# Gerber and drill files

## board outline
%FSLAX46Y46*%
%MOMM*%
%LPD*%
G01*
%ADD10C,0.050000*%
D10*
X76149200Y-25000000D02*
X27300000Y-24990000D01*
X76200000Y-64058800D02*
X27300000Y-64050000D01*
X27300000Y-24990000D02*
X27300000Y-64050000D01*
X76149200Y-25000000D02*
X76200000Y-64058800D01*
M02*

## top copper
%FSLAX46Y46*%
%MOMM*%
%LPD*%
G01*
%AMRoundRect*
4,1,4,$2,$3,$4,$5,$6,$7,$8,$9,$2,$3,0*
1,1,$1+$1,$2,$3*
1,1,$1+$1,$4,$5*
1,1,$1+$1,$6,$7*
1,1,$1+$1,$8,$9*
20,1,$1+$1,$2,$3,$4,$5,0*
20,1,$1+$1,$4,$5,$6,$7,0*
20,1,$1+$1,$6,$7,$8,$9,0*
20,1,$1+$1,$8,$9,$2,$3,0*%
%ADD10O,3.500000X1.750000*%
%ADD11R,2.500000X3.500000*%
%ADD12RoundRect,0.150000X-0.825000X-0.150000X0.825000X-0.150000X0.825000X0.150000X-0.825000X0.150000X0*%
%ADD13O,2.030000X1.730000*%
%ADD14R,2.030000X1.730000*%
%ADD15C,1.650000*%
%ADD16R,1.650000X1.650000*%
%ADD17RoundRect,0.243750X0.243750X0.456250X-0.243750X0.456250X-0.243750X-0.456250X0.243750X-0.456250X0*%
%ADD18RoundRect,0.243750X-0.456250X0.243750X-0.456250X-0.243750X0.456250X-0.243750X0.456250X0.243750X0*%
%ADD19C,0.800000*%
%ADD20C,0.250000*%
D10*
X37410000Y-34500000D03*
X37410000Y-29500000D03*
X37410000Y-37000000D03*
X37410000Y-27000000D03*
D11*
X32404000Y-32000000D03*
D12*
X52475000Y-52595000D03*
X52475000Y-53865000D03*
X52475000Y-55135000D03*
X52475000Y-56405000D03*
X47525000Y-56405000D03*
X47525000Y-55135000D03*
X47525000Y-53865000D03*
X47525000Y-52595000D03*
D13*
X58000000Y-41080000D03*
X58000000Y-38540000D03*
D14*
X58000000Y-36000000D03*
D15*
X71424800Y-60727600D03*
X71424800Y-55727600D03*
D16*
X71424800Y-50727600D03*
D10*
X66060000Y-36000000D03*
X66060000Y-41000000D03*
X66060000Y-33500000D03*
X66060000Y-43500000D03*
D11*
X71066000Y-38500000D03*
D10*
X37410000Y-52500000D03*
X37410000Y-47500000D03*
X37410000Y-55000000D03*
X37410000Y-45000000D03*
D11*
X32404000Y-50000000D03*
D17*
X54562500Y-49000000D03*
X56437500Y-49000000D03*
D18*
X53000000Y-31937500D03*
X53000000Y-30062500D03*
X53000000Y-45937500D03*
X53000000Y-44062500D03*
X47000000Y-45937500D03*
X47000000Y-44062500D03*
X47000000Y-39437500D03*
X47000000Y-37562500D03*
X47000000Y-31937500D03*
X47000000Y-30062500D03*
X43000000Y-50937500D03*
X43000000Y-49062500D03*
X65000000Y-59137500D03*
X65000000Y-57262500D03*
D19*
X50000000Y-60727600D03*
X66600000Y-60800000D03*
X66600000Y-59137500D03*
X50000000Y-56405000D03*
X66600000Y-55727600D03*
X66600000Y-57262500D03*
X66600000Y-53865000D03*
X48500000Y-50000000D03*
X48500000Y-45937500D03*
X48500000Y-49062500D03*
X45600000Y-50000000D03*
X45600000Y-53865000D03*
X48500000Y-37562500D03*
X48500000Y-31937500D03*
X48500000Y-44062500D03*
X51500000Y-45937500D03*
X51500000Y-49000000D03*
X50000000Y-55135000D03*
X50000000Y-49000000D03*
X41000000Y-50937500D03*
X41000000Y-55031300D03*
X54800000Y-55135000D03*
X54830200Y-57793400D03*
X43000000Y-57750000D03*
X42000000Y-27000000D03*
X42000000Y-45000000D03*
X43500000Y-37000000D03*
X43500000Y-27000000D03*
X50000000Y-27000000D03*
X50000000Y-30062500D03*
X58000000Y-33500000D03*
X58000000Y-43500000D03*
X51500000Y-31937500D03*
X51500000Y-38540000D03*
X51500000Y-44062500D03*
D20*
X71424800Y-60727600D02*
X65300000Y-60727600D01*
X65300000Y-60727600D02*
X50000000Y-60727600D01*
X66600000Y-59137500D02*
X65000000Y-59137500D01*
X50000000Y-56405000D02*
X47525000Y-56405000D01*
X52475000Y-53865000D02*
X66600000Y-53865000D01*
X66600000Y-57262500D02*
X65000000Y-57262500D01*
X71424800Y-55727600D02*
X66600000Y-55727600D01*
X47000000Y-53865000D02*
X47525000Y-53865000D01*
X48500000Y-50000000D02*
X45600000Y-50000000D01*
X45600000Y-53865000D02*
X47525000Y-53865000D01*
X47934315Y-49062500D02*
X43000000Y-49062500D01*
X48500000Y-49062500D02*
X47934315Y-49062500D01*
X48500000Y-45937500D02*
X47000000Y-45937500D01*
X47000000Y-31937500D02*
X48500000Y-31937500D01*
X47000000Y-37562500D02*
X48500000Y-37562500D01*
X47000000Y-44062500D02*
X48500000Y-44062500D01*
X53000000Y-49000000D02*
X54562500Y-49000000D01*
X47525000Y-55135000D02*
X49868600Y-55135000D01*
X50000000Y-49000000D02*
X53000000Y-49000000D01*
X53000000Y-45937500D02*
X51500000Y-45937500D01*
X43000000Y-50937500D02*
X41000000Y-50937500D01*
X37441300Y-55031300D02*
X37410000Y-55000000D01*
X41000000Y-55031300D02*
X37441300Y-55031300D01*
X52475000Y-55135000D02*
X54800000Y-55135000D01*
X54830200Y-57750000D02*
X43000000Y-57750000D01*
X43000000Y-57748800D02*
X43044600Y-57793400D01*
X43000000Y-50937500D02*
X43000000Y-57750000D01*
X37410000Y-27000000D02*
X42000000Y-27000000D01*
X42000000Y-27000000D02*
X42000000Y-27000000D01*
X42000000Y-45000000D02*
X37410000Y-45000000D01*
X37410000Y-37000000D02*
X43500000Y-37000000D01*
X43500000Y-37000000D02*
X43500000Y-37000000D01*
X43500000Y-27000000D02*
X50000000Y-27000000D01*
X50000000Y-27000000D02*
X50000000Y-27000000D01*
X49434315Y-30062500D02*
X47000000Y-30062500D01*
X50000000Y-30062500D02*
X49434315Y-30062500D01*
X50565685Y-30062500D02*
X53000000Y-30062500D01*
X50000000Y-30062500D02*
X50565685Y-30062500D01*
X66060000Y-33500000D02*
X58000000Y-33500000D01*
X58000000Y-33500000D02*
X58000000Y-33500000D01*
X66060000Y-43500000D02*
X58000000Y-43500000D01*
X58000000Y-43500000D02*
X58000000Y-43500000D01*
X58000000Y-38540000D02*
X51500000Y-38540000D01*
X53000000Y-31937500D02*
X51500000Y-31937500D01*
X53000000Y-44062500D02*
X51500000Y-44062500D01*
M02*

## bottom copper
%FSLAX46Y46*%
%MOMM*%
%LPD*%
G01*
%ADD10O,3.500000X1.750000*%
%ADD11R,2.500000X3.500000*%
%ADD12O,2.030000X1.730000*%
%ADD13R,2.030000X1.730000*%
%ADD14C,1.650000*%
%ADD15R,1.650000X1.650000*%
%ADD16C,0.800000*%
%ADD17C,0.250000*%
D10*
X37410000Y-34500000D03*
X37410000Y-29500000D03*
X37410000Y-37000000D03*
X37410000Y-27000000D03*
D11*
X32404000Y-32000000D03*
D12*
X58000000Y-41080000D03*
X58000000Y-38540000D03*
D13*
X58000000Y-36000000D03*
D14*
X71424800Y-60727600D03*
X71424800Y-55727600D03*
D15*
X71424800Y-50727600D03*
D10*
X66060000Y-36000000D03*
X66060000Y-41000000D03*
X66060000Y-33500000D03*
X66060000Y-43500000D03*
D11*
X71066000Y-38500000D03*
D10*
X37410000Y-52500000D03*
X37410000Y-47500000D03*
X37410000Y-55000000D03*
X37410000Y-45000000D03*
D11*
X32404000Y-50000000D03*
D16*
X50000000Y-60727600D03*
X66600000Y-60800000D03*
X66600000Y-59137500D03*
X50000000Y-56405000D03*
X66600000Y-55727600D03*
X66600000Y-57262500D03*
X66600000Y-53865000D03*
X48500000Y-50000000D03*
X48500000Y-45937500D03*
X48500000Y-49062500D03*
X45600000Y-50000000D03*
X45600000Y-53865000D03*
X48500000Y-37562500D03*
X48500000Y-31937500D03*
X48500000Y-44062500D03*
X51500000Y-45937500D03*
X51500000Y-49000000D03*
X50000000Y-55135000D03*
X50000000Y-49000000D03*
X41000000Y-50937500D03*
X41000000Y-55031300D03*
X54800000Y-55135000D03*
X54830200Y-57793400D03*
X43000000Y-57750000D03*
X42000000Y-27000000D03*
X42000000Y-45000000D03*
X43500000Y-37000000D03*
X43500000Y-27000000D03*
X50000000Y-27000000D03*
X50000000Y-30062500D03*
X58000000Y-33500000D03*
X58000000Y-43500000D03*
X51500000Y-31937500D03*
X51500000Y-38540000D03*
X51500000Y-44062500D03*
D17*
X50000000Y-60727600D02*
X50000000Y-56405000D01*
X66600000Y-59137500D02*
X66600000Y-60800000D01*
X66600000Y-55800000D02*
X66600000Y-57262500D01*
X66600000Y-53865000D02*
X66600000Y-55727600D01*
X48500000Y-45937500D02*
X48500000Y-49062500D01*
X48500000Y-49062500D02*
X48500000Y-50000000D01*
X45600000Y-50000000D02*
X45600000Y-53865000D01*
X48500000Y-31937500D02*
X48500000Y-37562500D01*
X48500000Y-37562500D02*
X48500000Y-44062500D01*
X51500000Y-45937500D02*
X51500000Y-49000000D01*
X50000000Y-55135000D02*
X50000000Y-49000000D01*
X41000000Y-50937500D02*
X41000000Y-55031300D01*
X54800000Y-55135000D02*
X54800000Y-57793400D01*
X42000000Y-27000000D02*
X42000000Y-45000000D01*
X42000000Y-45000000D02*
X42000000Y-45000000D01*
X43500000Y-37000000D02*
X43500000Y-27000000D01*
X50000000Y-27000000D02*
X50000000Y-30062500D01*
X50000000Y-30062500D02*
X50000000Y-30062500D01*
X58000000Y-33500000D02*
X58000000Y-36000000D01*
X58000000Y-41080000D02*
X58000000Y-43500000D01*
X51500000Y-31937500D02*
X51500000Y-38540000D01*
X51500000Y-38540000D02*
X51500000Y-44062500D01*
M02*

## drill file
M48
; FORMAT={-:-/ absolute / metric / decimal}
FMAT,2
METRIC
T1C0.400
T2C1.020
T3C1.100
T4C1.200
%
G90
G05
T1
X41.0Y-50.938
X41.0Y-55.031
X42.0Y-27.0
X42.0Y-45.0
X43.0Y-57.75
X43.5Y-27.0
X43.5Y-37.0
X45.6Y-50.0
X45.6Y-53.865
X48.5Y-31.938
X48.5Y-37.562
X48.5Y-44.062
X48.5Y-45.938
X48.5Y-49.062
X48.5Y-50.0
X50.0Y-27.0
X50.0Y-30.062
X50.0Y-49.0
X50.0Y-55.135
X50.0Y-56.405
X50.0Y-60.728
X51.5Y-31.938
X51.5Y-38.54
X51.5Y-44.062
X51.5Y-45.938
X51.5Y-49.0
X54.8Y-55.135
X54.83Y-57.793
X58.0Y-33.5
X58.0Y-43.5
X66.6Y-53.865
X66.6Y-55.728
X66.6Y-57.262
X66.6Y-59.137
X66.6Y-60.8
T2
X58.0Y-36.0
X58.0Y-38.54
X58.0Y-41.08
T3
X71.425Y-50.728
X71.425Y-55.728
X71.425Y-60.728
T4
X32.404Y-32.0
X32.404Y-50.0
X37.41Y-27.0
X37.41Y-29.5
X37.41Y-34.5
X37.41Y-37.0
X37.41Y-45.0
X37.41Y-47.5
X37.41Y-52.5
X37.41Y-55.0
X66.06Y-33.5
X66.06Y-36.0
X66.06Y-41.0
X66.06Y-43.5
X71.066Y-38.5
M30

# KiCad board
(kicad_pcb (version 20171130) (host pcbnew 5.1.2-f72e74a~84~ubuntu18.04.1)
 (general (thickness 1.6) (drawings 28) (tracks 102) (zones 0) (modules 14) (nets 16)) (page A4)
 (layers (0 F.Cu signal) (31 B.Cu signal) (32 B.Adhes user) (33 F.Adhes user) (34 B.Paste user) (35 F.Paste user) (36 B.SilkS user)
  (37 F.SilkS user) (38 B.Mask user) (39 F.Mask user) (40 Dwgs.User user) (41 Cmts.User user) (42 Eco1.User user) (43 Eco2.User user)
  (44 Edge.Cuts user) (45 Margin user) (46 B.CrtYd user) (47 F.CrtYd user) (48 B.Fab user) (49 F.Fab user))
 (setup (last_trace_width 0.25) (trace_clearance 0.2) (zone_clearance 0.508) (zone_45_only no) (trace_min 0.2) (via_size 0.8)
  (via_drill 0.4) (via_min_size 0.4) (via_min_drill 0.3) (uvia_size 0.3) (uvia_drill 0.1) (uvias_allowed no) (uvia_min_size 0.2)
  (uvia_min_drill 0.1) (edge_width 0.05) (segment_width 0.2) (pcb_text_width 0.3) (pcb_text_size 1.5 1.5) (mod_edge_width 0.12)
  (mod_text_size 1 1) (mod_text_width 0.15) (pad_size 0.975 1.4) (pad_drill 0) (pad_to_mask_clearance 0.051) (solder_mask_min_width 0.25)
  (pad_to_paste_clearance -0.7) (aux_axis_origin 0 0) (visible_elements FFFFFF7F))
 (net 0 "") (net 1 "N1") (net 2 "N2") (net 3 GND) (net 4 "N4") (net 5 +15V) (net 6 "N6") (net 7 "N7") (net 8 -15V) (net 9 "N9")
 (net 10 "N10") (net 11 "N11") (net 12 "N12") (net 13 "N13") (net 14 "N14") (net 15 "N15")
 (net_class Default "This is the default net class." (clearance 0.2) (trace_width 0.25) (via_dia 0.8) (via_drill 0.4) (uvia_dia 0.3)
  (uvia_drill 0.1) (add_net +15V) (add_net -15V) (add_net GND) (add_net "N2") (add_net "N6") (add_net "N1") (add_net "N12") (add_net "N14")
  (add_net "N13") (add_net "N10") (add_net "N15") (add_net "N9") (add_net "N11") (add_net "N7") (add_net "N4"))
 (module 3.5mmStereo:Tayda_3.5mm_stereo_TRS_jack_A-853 (layer F.Cu) (at 34 32 90)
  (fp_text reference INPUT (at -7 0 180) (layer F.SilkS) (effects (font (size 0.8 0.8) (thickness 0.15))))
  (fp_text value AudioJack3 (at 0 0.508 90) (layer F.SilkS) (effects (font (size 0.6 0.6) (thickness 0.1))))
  (pad 5 thru_hole oval (at -2.5 3.41 90) (size 1.75 3.5) (drill 1.2) (layers *.Cu *.Mask F.SilkS))
  (pad 4 thru_hole oval (at 2.5 3.41 90) (size 1.75 3.5) (drill 1.2) (layers *.Cu *.Mask F.SilkS))
  (pad 3 thru_hole oval (at -5 3.41 90) (size 1.75 3.5) (drill 1.2) (layers *.Cu *.Mask F.SilkS) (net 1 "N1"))
  (pad 2 thru_hole oval (at 5 3.41 90) (size 1.75 3.5) (drill 1.2) (layers *.Cu *.Mask F.SilkS) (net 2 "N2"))
  (pad 1 thru_hole rect (at 0 -1.596 90) (size 3.5 2.5) (drill 1.2) (layers *.Cu *.Mask F.SilkS) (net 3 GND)))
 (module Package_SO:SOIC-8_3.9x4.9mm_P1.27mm (layer F.Cu) (at 50 54.5)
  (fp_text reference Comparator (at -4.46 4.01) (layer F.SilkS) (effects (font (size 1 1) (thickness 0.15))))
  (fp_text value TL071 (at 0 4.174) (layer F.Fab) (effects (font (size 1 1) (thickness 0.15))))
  (pad 8 smd roundrect (at 2.475 -1.905) (size 1.95 0.6) (layers F.Cu F.Paste F.Mask) (roundrect_rratio 0.25) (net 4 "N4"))
  (pad 7 smd roundrect (at 2.475 -0.635) (size 1.95 0.6) (layers F.Cu F.Paste F.Mask) (roundrect_rratio 0.25) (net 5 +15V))
  (pad 6 smd roundrect (at 2.475 0.635) (size 1.95 0.6) (layers F.Cu F.Paste F.Mask) (roundrect_rratio 0.25) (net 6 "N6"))
  (pad 5 smd roundrect (at 2.475 1.905) (size 1.95 0.6) (layers F.Cu F.Paste F.Mask) (roundrect_rratio 0.25) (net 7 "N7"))
  (pad 4 smd roundrect (at -2.475 1.905) (size 1.95 0.6) (layers F.Cu F.Paste F.Mask) (roundrect_rratio 0.25) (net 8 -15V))
  (pad 3 smd roundrect (at -2.475 0.635) (size 1.95 0.6) (layers F.Cu F.Paste F.Mask) (roundrect_rratio 0.25) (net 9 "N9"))
  (pad 2 smd roundrect (at -2.475 -0.635) (size 1.95 0.6) (layers F.Cu F.Paste F.Mask) (roundrect_rratio 0.25) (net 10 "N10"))
  (pad 1 smd roundrect (at -2.475 -1.905) (size 1.95 0.6) (layers F.Cu F.Paste F.Mask) (roundrect_rratio 0.25) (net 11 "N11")))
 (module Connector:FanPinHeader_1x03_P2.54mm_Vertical (layer F.Cu) (at 58 36 270)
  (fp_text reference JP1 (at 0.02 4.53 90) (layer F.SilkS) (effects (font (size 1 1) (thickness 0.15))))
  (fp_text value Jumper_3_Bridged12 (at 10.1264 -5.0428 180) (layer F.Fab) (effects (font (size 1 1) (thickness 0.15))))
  (pad 3 thru_hole oval (at 5.08 0) (size 2.03 1.73) (drill 1.02) (layers *.Cu *.Mask) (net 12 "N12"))
  (pad 2 thru_hole oval (at 2.54 0) (size 2.03 1.73) (drill 1.02) (layers *.Cu *.Mask) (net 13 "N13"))
  (pad 1 thru_hole rect (at 0 0) (size 2.03 1.73) (drill 1.02) (layers *.Cu *.Mask) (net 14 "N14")))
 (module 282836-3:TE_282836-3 (layer F.Cu) (at 71.4248 55.7276 270)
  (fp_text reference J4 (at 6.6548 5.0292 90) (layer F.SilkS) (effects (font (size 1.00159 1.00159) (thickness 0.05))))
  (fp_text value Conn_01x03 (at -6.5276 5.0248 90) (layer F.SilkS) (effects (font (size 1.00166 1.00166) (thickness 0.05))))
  (pad 3 thru_hole circle (at 5 0 270) (size 1.65 1.65) (drill 1.1) (layers *.Cu *.Mask) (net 8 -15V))
  (pad 2 thru_hole circle (at 0 0 270) (size 1.65 1.65) (drill 1.1) (layers *.Cu *.Mask) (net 5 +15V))
  (pad 1 thru_hole rect (at -5 0 270) (size 1.65 1.65) (drill 1.1) (layers *.Cu *.Mask) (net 3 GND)))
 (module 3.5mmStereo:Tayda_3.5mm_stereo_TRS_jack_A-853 (layer F.Cu) (at 69.47 38.5 270)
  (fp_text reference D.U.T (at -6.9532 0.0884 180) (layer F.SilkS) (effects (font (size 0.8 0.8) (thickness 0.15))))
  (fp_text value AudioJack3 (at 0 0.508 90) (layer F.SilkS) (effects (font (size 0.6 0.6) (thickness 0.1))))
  (pad 5 thru_hole oval (at -2.5 3.41 270) (size 1.75 3.5) (drill 1.2) (layers *.Cu *.Mask F.SilkS))
  (pad 4 thru_hole oval (at 2.5 3.41 270) (size 1.75 3.5) (drill 1.2) (layers *.Cu *.Mask F.SilkS))
  (pad 3 thru_hole oval (at -5 3.41 270) (size 1.75 3.5) (drill 1.2) (layers *.Cu *.Mask F.SilkS) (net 14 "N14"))
  (pad 2 thru_hole oval (at 5 3.41 270) (size 1.75 3.5) (drill 1.2) (layers *.Cu *.Mask F.SilkS) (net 12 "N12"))
  (pad 1 thru_hole rect (at 0 -1.596 270) (size 3.5 2.5) (drill 1.2) (layers *.Cu *.Mask F.SilkS) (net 3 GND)))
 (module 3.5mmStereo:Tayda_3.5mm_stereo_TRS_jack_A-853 (layer F.Cu) (at 34 50 90)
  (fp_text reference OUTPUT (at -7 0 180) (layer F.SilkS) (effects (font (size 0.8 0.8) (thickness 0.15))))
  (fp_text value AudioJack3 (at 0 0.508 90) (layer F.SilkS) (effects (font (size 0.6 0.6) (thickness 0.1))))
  (pad 5 thru_hole oval (at -2.5 3.41 90) (size 1.75 3.5) (drill 1.2) (layers *.Cu *.Mask F.SilkS))
  (pad 4 thru_hole oval (at 2.5 3.41 90) (size 1.75 3.5) (drill 1.2) (layers *.Cu *.Mask F.SilkS))
  (pad 3 thru_hole oval (at -5 3.41 90) (size 1.75 3.5) (drill 1.2) (layers *.Cu *.Mask F.SilkS) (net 6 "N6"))
  (pad 2 thru_hole oval (at 5 3.41 90) (size 1.75 3.5) (drill 1.2) (layers *.Cu *.Mask F.SilkS) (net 2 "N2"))
  (pad 1 thru_hole rect (at 0 -1.596 90) (size 3.5 2.5) (drill 1.2) (layers *.Cu *.Mask F.SilkS) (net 3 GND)))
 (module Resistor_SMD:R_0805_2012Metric (layer F.Cu) (at 55.5 49 180)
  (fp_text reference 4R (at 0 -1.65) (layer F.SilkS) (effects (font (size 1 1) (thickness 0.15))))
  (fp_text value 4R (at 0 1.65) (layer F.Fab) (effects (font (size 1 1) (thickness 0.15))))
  (pad 2 smd roundrect (at 0.9375 0 180) (size 0.975 1.4) (layers F.Cu F.Paste F.Mask) (roundrect_rratio 0.25) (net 9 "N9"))
  (pad 1 smd roundrect (at -0.9375 0 180) (size 0.975 1.4) (layers F.Cu F.Paste F.Mask) (roundrect_rratio 0.25) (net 3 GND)))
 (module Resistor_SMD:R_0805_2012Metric (layer F.Cu) (at 53 31 270)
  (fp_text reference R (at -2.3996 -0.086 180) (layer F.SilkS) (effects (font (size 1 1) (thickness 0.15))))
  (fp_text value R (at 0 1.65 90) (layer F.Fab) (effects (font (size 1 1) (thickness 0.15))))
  (pad 2 smd roundrect (at 0.9375 0 270) (size 0.975 1.4) (layers F.Cu F.Paste F.Mask) (roundrect_rratio 0.25) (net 13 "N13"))
  (pad 1 smd roundrect (at -0.9375 0 270) (size 0.975 1.4) (layers F.Cu F.Paste F.Mask) (roundrect_rratio 0.25) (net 1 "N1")))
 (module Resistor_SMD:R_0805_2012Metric (layer F.Cu) (at 53 45 270)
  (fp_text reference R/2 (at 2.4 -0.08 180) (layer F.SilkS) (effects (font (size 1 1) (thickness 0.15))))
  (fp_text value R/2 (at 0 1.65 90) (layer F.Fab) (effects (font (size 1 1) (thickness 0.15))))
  (pad 2 smd roundrect (at 0.9375 0 270) (size 0.975 1.4) (layers F.Cu F.Paste F.Mask) (roundrect_rratio 0.25) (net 9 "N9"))
  (pad 1 smd roundrect (at -0.9375 0 270) (size 0.975 1.4) (layers F.Cu F.Paste F.Mask) (roundrect_rratio 0.25) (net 13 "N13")))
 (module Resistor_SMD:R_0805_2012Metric (layer F.Cu) (at 47 45 270)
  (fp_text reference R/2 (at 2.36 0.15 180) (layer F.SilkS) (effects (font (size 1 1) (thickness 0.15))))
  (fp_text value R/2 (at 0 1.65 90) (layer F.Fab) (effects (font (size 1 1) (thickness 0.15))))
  (pad 2 smd roundrect (at 0.9375 0 270) (size 0.975 1.4) (layers F.Cu F.Paste F.Mask) (roundrect_rratio 0.25) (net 10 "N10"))
  (pad 1 smd roundrect (at -0.9375 0 270) (size 0.975 1.4) (layers F.Cu F.Paste F.Mask) (roundrect_rratio 0.25) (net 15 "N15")))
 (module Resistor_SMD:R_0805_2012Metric (layer F.Cu) (at 47 38.5 270)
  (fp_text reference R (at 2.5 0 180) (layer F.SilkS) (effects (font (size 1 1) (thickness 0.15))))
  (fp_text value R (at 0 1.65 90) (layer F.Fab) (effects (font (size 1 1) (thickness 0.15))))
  (pad 2 smd roundrect (at 0.9375 0 270) (size 0.975 1.4) (layers F.Cu F.Paste F.Mask) (roundrect_rratio 0.25) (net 3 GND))
  (pad 1 smd roundrect (at -0.9375 0 270) (size 0.975 1.4) (layers F.Cu F.Paste F.Mask) (roundrect_rratio 0.25) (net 15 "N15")))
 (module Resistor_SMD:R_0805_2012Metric (layer F.Cu) (at 47 31 270)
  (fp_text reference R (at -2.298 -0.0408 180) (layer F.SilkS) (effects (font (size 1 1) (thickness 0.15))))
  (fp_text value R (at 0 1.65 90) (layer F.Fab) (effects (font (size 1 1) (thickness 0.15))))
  (pad 2 smd roundrect (at 0.9375 0 270) (size 0.975 1.4) (layers F.Cu F.Paste F.Mask) (roundrect_rratio 0.25) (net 15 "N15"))
  (pad 1 smd roundrect (at -0.9375 0 270) (size 0.975 1.4) (layers F.Cu F.Paste F.Mask) (roundrect_rratio 0.25) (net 1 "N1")))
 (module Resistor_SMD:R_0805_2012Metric (layer F.Cu) (at 43 50 270)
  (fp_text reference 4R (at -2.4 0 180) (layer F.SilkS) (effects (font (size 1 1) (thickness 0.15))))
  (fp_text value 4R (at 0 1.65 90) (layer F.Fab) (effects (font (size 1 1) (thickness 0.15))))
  (pad 2 smd roundrect (at 0.9375 0 270) (size 0.975 1.4) (layers F.Cu F.Paste F.Mask) (roundrect_rratio 0.25) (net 6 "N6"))
  (pad 1 smd roundrect (at -0.9375 0 270) (size 0.975 1.4) (layers F.Cu F.Paste F.Mask) (roundrect_rratio 0.25) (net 10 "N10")))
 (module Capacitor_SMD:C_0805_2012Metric (layer F.Cu) (at 65 58.2 270)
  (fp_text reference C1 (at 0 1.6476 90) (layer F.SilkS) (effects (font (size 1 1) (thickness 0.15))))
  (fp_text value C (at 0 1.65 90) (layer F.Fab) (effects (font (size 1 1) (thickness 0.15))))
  (pad 2 smd roundrect (at 0.9375 0 270) (size 0.975 1.4) (layers F.Cu F.Paste F.Mask) (roundrect_rratio 0.25) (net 8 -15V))
  (pad 1 smd roundrect (at -0.9375 0 270) (size 0.975 1.4) (layers F.Cu F.Paste F.Mask) (roundrect_rratio 0.25) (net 5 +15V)))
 (gr_line (start 76.1492 25) (end 27.3 24.99) (layer Edge.Cuts) (width 0.05))
 (gr_line (start 76.2 64.0588) (end 27.3 64.05) (layer Edge.Cuts) (width 0.05))
 (gr_line (start 27.3 24.99) (end 27.3 64.05) (layer Edge.Cuts) (width 0.05))
 (gr_line (start 76.1492 25) (end 76.2 64.0588) (layer Edge.Cuts) (width 0.05))
 (via (at 50 60.7276) (size 0.8) (drill 0.4) (layers F.Cu B.Cu) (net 8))
 (segment (start 71.4248 60.7276) (end 65.3 60.7276) (width 0.25) (layer F.Cu) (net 8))
 (via (at 66.6 60.8) (size 0.8) (drill 0.4) (layers F.Cu B.Cu) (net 8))
 (via (at 66.6 59.1375) (size 0.8) (drill 0.4) (layers F.Cu B.Cu) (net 8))
 (segment (start 65.3 60.7276) (end 50 60.7276) (width 0.25) (layer F.Cu) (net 8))
 (segment (start 50 60.7276) (end 50 56.405) (width 0.25) (layer B.Cu) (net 8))
 (via (at 50 56.405) (size 0.8) (drill 0.4) (layers F.Cu B.Cu) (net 8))
 (segment (start 66.6 59.1375) (end 66.6 60.8) (width 0.25) (layer B.Cu) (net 8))
 (segment (start 66.6 59.1375) (end 65 59.1375) (width 0.25) (layer F.Cu) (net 8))
 (segment (start 50 56.405) (end 47.525 56.405) (width 0.25) (layer F.Cu) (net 8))
 (via (at 66.6 55.7276) (size 0.8) (drill 0.4) (layers F.Cu B.Cu) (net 5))
 (segment (start 66.6 55.8) (end 66.6 57.2625) (width 0.25) (layer B.Cu) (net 5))
 (via (at 66.6 57.2625) (size 0.8) (drill 0.4) (layers F.Cu B.Cu) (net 5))
 (segment (start 52.475 53.865) (end 66.6 53.865) (width 0.25) (layer F.Cu) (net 5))
 (via (at 66.6 53.865) (size 0.8) (drill 0.4) (layers F.Cu B.Cu) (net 5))
 (segment (start 66.6 53.865) (end 66.6 55.7276) (width 0.25) (layer B.Cu) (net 5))
 (segment (start 66.6 57.2625) (end 65 57.2625) (width 0.25) (layer F.Cu) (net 5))
 (segment (start 71.4248 55.7276) (end 66.6 55.7276) (width 0.25) (layer F.Cu) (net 5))
 (via (at 48.5 50) (size 0.8) (drill 0.4) (layers F.Cu B.Cu) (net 10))
 (via (at 48.5 45.9375) (size 0.8) (drill 0.4) (layers F.Cu B.Cu) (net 10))
 (segment (start 48.5 45.9375) (end 48.5 49.0625) (width 0.25) (layer B.Cu) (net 10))
 (via (at 48.5 49.0625) (size 0.8) (drill 0.4) (layers F.Cu B.Cu) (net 10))
 (segment (start 47 53.865) (end 47.525 53.865) (width 0.25) (layer F.Cu) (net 10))
 (segment (start 48.5 49.0625) (end 48.5 50) (width 0.25) (layer B.Cu) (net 10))
 (segment (start 48.5 50) (end 45.6 50) (width 0.25) (layer F.Cu) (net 10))
 (via (at 45.6 50) (size 0.8) (drill 0.4) (layers F.Cu B.Cu) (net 10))
 (segment (start 45.6 50) (end 45.6 53.865) (width 0.25) (layer B.Cu) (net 10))
 (via (at 45.6 53.865) (size 0.8) (drill 0.4) (layers F.Cu B.Cu) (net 10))
 (segment (start 45.6 53.865) (end 47.525 53.865) (width 0.25) (layer F.Cu) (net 10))
 (segment (start 47.934315 49.0625) (end 43 49.0625) (width 0.25) (layer F.Cu) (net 10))
 (segment (start 48.5 49.0625) (end 47.934315 49.0625) (width 0.25) (layer F.Cu) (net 10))
 (segment (start 48.5 45.9375) (end 47 45.9375) (width 0.25) (layer F.Cu) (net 10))
 (via (at 48.5 37.5625) (size 0.8) (drill 0.4) (layers F.Cu B.Cu) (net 15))
 (via (at 48.5 31.9375) (size 0.8) (drill 0.4) (layers F.Cu B.Cu) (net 15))
 (segment (start 48.5 31.9375) (end 48.5 37.5625) (width 0.25) (layer B.Cu) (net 15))
 (segment (start 48.5 37.5625) (end 48.5 44.0625) (width 0.25) (layer B.Cu) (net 15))
 (via (at 48.5 44.0625) (size 0.8) (drill 0.4) (layers F.Cu B.Cu) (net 15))
 (segment (start 47 31.9375) (end 48.5 31.9375) (width 0.25) (layer F.Cu) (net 15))
 (segment (start 47 37.5625) (end 48.5 37.5625) (width 0.25) (layer F.Cu) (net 15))
 (segment (start 47 44.0625) (end 48.5 44.0625) (width 0.25) (layer F.Cu) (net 15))
 (via (at 51.5 45.9375) (size 0.8) (drill 0.4) (layers F.Cu B.Cu) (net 9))
 (segment (start 51.5 45.9375) (end 51.5 49) (width 0.25) (layer B.Cu) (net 9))
 (via (at 51.5 49) (size 0.8) (drill 0.4) (layers F.Cu B.Cu) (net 9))
 (segment (start 53 49) (end 54.5625 49) (width 0.25) (layer F.Cu) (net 9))
 (segment (start 47.525 55.135) (end 49.8686 55.135) (width 0.25) (layer F.Cu) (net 9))
 (via (at 50 55.135) (size 0.8) (drill 0.4) (layers F.Cu B.Cu) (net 9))
 (segment (start 50 55.135) (end 50 49) (width 0.25) (layer B.Cu) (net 9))
 (via (at 50 49) (size 0.8) (drill 0.4) (layers F.Cu B.Cu) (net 9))
 (segment (start 50 49) (end 53 49) (width 0.25) (layer F.Cu) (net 9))
 (segment (start 53 45.9375) (end 51.5 45.9375) (width 0.25) (layer F.Cu) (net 9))
 (segment (start 43 50.9375) (end 41 50.9375) (width 0.25) (layer F.Cu) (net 6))
 (via (at 41 50.9375) (size 0.8) (drill 0.4) (layers F.Cu B.Cu) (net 6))
 (segment (start 41 50.9375) (end 41 55.0313) (width 0.25) (layer B.Cu) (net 6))
 (via (at 41 55.0313) (size 0.8) (drill 0.4) (layers F.Cu B.Cu) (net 6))
 (segment (start 37.4413 55.0313) (end 37.41 55) (width 0.25) (layer F.Cu) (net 6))
 (segment (start 41 55.0313) (end 37.4413 55.0313) (width 0.25) (layer F.Cu) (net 6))
 (segment (start 52.475 55.135) (end 54.8 55.135) (width 0.25) (layer F.Cu) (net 6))
 (via (at 54.8 55.135) (size 0.8) (drill 0.4) (layers F.Cu B.Cu) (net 6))
 (segment (start 54.8 55.135) (end 54.8 57.7934) (width 0.25) (layer B.Cu) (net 6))
 (via (at 54.8302 57.7934) (size 0.8) (drill 0.4) (layers F.Cu B.Cu) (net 6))
 (segment (start 54.8302 57.75) (end 43 57.75) (width 0.25) (layer F.Cu) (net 6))
 (via (at 43 57.75) (size 0.8) (drill 0.4) (layers F.Cu B.Cu) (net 6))
 (segment (start 43 57.7488) (end 43.0446 57.7934) (width 0.25) (layer F.Cu) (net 6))
 (segment (start 43 50.9375) (end 43 57.75) (width 0.25) (layer F.Cu) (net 6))
 (segment (start 37.41 27) (end 42 27) (width 0.25) (layer F.Cu) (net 2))
 (segment (start 42 27) (end 42 27) (width 0.25) (layer F.Cu) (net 2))
 (via (at 42 27) (size 0.8) (drill 0.4) (layers F.Cu B.Cu) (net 2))
 (segment (start 42 27) (end 42 45) (width 0.25) (layer B.Cu) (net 2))
 (segment (start 42 45) (end 42 45) (width 0.25) (layer B.Cu) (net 2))
 (via (at 42 45) (size 0.8) (drill 0.4) (layers F.Cu B.Cu) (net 2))
 (segment (start 42 45) (end 37.41 45) (width 0.25) (layer F.Cu) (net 2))
 (segment (start 37.41 37) (end 43.5 37) (width 0.25) (layer F.Cu) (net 1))
 (segment (start 43.5 37) (end 43.5 37) (width 0.25) (layer F.Cu) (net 1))
 (via (at 43.5 37) (size 0.8) (drill 0.4) (layers F.Cu B.Cu) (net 1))
 (segment (start 43.5 37) (end 43.5 27) (width 0.25) (layer B.Cu) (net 1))
 (via (at 43.5 27) (size 0.8) (drill 0.4) (layers F.Cu B.Cu) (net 1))
 (segment (start 43.5 27) (end 50 27) (width 0.25) (layer F.Cu) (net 1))
 (segment (start 50 27) (end 50 27) (width 0.25) (layer F.Cu) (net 1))
 (via (at 50 27) (size 0.8) (drill 0.4) (layers F.Cu B.Cu) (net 1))
 (segment (start 50 27) (end 50 30.0625) (width 0.25) (layer B.Cu) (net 1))
 (segment (start 50 30.0625) (end 50 30.0625) (width 0.25) (layer B.Cu) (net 1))
 (via (at 50 30.0625) (size 0.8) (drill 0.4) (layers F.Cu B.Cu) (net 1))
 (segment (start 49.434315 30.0625) (end 47 30.0625) (width 0.25) (layer F.Cu) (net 1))
 (segment (start 50 30.0625) (end 49.434315 30.0625) (width 0.25) (layer F.Cu) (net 1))
 (segment (start 50.565685 30.0625) (end 53 30.0625) (width 0.25) (layer F.Cu) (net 1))
 (segment (start 50 30.0625) (end 50.565685 30.0625) (width 0.25) (layer F.Cu) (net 1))
 (segment (start 66.06 33.5) (end 58 33.5) (width 0.25) (layer F.Cu) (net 14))
 (segment (start 58 33.5) (end 58 33.5) (width 0.25) (layer F.Cu) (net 14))
 (via (at 58 33.5) (size 0.8) (drill 0.4) (layers F.Cu B.Cu) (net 14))
 (segment (start 58 33.5) (end 58 36) (width 0.25) (layer B.Cu) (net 14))
 (segment (start 66.06 43.5) (end 58 43.5) (width 0.25) (layer F.Cu) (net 12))
 (segment (start 58 43.5) (end 58 43.5) (width 0.25) (layer F.Cu) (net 12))
 (via (at 58 43.5) (size 0.8) (drill 0.4) (layers F.Cu B.Cu) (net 12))
 (segment (start 58 41.08) (end 58 43.5) (width 0.25) (layer B.Cu) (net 12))
 (via (at 51.5 31.9375) (size 0.8) (drill 0.4) (layers F.Cu B.Cu) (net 13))
 (segment (start 51.5 31.9375) (end 51.5 38.54) (width 0.25) (layer B.Cu) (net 13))
 (via (at 51.5 38.54) (size 0.8) (drill 0.4) (layers F.Cu B.Cu) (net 13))
 (segment (start 51.5 38.54) (end 51.5 44.0625) (width 0.25) (layer B.Cu) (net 13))
 (via (at 51.5 44.0625) (size 0.8) (drill 0.4) (layers F.Cu B.Cu) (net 13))
 (segment (start 58 38.54) (end 51.5 38.54) (width 0.25) (layer F.Cu) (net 13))
 (segment (start 53 31.9375) (end 51.5 31.9375) (width 0.25) (layer F.Cu) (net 13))
 (segment (start 53 44.0625) (end 51.5 44.0625) (width 0.25) (layer F.Cu) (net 13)))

